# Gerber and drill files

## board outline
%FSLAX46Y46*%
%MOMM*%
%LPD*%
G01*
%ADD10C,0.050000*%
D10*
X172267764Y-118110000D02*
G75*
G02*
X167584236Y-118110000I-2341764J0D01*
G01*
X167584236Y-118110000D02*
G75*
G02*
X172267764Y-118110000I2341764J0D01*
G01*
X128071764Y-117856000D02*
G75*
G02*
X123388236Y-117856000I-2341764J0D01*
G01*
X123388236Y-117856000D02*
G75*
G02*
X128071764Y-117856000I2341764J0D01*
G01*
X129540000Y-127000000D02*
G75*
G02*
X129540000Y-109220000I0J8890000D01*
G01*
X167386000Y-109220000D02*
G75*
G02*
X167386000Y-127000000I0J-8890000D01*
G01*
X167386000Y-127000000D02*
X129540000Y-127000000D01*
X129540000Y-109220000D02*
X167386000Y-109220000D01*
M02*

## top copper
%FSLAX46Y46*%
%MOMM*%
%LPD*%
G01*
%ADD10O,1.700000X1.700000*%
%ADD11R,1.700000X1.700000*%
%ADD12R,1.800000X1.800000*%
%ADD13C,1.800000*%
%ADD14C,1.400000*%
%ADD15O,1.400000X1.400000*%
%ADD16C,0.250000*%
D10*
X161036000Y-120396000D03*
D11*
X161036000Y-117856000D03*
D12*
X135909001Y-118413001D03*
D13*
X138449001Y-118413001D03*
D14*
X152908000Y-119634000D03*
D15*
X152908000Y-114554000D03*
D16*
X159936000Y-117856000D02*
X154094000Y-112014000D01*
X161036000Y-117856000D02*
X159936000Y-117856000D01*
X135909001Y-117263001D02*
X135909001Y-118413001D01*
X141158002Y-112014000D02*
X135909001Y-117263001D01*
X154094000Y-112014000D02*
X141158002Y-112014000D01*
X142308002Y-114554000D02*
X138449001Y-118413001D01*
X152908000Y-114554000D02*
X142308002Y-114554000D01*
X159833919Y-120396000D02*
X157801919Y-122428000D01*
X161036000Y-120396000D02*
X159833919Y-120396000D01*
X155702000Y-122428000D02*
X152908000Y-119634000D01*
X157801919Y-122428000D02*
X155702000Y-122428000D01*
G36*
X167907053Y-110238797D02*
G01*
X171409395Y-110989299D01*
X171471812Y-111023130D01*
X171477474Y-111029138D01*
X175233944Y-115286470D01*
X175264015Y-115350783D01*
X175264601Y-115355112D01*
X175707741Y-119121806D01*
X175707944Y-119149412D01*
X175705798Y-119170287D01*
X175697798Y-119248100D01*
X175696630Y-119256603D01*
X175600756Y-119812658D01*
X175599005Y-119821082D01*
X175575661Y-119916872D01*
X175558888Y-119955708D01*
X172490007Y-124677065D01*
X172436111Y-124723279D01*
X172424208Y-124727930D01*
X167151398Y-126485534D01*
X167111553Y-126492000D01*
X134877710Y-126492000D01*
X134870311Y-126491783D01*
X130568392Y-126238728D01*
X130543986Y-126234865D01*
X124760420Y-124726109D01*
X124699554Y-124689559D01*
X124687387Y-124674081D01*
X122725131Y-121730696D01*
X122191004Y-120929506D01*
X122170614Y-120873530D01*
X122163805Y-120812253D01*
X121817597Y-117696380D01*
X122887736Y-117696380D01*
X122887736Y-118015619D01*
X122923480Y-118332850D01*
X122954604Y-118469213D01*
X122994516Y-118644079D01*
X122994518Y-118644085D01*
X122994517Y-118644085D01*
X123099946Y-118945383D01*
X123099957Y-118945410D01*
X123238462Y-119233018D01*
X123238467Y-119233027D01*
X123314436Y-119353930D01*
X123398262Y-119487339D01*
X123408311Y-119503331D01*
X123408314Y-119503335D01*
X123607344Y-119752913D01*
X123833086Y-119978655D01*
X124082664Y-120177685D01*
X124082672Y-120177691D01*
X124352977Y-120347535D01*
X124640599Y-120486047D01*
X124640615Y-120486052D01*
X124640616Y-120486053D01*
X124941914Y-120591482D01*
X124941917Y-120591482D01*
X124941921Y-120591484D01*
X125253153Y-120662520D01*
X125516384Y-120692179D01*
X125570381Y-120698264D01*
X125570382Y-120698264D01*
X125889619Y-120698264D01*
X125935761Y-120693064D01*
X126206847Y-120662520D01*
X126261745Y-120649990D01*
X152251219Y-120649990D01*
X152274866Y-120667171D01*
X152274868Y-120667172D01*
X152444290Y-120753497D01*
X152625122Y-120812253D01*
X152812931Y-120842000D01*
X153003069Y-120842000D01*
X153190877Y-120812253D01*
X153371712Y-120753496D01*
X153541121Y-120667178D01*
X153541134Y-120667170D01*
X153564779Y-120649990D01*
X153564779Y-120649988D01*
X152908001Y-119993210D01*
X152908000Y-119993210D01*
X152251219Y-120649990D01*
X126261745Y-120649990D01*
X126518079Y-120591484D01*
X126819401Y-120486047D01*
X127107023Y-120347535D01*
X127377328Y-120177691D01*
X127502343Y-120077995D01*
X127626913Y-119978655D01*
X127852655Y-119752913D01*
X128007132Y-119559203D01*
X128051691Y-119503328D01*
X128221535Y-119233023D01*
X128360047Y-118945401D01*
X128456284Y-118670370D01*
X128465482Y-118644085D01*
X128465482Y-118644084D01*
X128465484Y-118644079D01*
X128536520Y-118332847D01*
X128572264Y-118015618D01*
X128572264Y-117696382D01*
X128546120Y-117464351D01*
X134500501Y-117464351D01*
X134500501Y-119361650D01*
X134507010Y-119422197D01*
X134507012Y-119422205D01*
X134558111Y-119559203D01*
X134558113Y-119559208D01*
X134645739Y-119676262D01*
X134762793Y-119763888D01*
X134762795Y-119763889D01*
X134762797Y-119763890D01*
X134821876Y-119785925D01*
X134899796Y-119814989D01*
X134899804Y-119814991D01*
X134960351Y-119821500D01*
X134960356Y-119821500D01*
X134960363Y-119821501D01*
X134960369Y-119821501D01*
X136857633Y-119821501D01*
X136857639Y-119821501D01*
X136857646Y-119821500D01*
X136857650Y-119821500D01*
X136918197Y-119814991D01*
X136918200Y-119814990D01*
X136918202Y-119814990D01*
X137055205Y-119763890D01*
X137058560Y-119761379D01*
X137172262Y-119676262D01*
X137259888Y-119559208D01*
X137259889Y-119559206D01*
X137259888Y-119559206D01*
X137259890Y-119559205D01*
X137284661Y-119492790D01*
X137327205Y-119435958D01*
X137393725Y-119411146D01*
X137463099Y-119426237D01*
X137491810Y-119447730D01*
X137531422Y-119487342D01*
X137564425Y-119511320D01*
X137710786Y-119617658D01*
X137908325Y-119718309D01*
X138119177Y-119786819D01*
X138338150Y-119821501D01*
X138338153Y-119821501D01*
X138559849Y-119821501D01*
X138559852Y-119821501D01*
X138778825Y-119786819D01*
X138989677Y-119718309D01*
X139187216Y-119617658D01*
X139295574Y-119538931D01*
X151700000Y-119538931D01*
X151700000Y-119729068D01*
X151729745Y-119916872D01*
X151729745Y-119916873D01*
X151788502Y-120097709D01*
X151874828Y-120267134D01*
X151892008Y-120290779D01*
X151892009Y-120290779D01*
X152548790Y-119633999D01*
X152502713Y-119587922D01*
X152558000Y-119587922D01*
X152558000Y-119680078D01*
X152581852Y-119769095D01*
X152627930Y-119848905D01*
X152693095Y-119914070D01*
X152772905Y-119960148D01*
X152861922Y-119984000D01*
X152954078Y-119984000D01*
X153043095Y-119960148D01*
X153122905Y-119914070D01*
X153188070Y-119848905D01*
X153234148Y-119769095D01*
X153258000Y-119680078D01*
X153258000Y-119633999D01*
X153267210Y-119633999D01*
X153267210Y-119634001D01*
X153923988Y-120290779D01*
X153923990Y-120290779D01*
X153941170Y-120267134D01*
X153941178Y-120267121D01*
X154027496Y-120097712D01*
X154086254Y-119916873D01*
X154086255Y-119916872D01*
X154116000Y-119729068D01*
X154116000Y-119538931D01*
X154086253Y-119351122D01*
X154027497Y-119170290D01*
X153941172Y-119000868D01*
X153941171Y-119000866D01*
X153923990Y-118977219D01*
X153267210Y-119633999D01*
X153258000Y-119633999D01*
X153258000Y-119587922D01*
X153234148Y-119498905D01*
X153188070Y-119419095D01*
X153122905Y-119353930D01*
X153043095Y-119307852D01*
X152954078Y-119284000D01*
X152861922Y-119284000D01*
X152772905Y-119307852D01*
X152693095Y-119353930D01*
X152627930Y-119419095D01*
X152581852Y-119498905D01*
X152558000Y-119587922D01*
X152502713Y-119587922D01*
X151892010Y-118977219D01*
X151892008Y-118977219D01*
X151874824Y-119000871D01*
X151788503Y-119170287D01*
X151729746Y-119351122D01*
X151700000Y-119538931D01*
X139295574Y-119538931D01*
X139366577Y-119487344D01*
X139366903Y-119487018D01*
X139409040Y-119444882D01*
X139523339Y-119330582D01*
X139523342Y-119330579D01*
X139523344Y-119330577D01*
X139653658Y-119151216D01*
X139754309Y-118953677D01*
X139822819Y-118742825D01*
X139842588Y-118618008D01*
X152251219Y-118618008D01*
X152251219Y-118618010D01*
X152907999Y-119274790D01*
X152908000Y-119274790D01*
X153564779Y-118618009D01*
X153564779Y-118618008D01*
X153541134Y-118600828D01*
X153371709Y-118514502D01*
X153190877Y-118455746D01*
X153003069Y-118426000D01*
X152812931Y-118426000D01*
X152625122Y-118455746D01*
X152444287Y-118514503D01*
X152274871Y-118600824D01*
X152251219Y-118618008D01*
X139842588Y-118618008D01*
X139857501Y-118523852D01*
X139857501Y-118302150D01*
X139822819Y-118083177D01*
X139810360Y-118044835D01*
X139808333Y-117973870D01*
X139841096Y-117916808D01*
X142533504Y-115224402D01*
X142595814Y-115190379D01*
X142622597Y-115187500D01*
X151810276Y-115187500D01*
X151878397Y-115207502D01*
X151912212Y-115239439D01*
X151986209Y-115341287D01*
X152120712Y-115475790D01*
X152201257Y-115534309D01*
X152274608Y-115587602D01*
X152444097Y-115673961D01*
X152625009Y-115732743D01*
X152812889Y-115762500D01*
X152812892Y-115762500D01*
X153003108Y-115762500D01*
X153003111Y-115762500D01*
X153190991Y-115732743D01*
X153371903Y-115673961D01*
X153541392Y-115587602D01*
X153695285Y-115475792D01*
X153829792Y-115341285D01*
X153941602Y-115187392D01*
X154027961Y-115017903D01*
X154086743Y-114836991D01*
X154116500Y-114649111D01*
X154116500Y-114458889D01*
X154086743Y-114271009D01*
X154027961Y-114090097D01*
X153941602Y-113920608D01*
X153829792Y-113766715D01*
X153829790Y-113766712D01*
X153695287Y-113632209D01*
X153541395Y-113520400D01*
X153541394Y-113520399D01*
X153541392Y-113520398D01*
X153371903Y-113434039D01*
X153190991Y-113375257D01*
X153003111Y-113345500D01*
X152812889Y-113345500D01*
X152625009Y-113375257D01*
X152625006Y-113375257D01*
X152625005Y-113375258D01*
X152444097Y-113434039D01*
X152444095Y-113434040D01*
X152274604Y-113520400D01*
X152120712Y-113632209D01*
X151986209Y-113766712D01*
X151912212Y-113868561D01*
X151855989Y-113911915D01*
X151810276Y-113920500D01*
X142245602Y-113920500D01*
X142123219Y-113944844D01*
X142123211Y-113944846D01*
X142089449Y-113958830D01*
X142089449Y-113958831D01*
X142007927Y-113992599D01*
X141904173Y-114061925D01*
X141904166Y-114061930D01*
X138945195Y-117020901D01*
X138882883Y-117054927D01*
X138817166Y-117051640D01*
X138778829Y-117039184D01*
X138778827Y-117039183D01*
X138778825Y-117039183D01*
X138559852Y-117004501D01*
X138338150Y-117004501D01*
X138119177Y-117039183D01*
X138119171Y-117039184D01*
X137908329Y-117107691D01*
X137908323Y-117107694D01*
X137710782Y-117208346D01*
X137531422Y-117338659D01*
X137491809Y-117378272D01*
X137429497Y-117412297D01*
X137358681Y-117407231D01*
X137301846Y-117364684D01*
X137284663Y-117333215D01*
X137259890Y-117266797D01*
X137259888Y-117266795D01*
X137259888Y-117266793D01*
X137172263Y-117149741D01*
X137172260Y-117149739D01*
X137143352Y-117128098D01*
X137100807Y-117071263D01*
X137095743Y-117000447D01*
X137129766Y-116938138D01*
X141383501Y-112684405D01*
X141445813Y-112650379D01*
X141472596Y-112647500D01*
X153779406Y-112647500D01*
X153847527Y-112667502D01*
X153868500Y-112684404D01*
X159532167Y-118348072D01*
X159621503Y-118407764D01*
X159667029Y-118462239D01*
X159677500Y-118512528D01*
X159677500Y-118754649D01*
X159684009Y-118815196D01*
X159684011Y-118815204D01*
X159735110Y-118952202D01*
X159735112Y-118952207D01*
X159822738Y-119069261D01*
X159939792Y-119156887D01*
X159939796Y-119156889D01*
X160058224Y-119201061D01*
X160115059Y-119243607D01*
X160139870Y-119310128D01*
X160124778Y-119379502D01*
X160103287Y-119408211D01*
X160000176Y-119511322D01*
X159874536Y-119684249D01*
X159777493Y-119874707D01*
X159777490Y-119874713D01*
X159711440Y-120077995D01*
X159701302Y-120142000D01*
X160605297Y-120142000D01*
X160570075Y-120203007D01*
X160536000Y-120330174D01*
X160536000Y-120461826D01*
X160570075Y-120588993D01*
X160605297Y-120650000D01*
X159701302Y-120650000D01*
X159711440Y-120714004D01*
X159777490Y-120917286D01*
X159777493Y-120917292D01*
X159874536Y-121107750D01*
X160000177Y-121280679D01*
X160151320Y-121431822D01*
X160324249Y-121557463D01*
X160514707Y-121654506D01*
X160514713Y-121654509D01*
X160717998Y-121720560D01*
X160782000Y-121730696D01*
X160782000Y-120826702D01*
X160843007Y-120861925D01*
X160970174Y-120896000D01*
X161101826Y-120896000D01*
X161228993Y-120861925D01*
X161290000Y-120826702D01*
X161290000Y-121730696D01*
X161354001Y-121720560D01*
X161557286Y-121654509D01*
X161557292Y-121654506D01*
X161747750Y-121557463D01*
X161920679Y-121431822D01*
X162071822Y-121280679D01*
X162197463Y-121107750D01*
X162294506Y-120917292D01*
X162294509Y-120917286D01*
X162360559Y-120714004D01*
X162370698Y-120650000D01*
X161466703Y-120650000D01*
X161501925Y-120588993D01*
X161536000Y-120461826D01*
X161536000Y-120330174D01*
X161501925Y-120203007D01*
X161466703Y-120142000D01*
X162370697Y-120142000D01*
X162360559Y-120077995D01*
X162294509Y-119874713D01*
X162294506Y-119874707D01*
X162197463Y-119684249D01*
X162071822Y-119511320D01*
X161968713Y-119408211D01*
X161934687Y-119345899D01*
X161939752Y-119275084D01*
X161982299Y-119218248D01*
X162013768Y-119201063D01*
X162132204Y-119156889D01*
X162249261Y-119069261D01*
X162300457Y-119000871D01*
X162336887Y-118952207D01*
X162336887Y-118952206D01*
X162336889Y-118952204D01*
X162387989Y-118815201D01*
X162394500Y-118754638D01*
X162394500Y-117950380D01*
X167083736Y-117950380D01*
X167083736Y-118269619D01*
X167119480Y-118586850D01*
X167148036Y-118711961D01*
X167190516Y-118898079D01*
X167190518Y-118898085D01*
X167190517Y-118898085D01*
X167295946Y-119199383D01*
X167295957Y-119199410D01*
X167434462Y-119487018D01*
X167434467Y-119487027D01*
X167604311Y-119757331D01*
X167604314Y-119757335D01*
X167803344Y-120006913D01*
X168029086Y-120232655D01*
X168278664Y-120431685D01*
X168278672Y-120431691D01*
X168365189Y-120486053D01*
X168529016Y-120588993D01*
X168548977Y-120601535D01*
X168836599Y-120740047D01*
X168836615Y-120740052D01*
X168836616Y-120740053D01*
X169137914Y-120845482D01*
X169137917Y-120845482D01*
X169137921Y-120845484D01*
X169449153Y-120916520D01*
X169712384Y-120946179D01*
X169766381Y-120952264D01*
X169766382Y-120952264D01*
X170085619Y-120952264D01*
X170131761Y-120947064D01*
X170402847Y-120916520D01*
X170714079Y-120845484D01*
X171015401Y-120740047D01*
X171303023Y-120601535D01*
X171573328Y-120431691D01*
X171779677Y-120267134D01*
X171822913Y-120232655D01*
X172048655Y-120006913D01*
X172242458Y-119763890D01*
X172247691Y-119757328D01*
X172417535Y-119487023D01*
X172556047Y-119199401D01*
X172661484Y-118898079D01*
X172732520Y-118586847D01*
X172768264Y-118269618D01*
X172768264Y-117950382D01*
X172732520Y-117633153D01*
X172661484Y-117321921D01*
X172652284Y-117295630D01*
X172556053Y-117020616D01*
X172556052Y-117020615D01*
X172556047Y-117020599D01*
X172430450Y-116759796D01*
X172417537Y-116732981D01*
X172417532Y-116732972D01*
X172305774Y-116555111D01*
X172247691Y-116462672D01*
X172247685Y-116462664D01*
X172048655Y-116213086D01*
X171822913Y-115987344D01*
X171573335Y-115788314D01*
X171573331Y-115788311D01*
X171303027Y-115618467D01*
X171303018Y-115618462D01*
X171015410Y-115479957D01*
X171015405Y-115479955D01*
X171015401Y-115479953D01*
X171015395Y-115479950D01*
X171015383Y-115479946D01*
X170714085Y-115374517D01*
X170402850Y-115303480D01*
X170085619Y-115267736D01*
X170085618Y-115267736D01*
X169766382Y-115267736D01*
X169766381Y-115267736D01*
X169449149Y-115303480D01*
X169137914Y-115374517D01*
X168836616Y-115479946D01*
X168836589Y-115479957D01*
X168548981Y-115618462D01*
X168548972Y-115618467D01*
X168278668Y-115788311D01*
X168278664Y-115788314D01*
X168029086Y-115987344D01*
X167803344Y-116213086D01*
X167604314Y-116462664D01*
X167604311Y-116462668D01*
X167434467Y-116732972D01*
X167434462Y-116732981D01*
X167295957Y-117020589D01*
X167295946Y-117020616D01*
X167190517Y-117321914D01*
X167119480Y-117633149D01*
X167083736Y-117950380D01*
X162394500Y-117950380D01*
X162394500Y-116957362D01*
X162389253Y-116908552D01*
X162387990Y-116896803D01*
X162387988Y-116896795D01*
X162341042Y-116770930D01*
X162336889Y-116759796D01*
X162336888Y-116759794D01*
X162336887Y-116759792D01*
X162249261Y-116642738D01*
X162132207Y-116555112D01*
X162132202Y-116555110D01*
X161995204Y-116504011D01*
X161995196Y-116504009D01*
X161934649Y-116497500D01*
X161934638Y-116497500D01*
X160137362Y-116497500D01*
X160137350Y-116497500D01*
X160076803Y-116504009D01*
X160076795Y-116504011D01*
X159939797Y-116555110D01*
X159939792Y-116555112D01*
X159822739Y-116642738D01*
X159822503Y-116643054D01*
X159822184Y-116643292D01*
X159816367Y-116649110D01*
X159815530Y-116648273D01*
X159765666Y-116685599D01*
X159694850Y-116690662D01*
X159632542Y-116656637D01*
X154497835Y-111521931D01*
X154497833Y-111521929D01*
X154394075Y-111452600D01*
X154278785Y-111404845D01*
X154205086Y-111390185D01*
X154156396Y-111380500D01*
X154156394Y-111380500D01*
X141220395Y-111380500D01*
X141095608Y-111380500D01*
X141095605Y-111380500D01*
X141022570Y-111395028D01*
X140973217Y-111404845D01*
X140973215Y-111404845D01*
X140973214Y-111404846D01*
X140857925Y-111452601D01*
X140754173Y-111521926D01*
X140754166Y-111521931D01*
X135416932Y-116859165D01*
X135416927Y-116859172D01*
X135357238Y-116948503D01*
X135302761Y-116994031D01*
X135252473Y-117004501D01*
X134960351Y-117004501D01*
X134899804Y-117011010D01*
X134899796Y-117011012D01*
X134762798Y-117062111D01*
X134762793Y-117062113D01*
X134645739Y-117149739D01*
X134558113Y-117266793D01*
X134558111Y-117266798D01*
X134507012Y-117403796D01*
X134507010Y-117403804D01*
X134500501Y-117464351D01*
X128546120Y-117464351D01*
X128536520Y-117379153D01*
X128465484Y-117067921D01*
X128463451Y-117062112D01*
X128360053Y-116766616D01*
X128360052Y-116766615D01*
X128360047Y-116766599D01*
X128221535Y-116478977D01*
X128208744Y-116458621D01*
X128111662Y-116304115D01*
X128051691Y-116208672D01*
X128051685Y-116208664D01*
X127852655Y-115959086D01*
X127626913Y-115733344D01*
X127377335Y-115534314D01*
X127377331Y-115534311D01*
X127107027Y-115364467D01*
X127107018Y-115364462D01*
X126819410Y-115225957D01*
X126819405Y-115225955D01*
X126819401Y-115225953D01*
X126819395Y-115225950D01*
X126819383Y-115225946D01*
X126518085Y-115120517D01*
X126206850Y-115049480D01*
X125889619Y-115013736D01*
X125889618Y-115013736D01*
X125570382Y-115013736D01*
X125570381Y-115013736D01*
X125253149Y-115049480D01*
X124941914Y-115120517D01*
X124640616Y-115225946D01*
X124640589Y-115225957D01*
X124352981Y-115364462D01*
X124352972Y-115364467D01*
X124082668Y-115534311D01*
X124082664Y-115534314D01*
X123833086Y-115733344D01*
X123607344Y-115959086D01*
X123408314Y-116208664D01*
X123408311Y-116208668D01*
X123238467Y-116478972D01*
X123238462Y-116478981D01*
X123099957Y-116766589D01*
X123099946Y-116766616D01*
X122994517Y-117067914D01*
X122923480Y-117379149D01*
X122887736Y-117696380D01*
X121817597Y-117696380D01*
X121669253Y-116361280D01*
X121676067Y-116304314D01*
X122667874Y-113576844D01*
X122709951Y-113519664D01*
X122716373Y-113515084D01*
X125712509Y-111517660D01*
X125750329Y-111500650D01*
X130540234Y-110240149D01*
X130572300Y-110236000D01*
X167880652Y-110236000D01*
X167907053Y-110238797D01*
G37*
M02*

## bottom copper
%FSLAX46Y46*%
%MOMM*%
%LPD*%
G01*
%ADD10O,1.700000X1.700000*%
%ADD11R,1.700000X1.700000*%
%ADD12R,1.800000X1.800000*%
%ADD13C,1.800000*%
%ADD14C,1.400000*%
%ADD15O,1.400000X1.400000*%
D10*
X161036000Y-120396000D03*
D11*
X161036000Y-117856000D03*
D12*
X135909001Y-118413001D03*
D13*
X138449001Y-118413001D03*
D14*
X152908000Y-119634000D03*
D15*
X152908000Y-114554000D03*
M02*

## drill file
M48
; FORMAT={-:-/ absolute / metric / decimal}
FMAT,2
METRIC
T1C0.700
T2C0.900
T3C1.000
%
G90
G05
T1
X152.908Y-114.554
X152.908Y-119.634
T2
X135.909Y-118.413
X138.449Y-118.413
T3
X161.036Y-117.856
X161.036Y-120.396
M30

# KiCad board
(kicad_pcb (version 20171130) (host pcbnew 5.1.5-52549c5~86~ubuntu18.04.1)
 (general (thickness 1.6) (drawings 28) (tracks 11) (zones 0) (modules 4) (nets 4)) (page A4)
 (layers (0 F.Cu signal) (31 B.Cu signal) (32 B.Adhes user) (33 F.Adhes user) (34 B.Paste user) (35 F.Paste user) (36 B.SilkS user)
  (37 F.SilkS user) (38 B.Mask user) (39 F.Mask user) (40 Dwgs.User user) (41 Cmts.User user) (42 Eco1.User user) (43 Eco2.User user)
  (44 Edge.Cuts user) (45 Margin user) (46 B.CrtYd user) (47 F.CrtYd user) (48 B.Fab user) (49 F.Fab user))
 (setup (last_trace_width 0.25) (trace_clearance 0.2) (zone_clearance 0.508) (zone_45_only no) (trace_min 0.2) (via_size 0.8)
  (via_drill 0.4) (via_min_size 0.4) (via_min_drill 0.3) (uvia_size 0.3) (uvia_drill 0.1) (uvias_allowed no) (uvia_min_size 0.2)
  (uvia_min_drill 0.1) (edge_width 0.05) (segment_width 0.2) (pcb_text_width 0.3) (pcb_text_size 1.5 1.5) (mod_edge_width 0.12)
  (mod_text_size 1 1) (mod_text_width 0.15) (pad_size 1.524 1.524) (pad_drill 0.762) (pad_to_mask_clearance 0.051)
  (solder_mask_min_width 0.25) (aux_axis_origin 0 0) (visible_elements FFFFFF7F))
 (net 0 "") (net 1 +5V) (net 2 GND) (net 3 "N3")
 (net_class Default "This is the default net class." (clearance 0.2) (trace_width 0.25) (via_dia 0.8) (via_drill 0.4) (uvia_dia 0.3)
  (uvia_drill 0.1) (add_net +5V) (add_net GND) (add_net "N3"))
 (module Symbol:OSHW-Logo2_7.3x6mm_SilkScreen (layer B.Cu) (at 146.558 121.158)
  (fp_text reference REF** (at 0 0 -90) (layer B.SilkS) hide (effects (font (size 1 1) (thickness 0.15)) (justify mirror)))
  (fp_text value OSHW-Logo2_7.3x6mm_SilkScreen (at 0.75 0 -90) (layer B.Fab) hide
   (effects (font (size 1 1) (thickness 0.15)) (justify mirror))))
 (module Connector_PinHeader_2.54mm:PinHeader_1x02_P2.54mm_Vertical (layer F.Cu) (at 161.036 117.856)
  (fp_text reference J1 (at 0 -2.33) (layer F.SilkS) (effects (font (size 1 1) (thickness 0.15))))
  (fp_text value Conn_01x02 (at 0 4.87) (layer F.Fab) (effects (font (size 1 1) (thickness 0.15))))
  (pad 2 thru_hole oval (at 0 2.54) (size 1.7 1.7) (drill 1) (layers *.Cu *.Mask) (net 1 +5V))
  (pad 1 thru_hole rect (at 0 0) (size 1.7 1.7) (drill 1) (layers *.Cu *.Mask) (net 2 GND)))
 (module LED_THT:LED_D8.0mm (layer F.Cu) (at 135.909001 118.413001)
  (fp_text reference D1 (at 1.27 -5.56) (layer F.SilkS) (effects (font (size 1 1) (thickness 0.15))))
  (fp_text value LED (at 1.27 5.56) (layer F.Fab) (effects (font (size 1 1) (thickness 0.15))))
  (pad 1 thru_hole rect (at 0 0) (size 1.8 1.8) (drill 0.9) (layers *.Cu *.Mask) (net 2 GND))
  (pad 2 thru_hole circle (at 2.54 0) (size 1.8 1.8) (drill 0.9) (layers *.Cu *.Mask) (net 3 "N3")))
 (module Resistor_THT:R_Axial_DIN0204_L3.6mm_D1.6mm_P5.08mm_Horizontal (layer F.Cu) (at 152.908 119.634 90)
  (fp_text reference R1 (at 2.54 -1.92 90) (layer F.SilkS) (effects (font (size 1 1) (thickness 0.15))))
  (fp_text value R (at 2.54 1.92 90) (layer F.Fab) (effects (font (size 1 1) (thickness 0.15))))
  (pad 1 thru_hole circle (at 0 0 90) (size 1.4 1.4) (drill 0.7) (layers *.Cu *.Mask) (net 1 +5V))
  (pad 2 thru_hole oval (at 5.08 0 90) (size 1.4 1.4) (drill 0.7) (layers *.Cu *.Mask) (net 3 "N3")))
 (gr_circle (center 169.926 118.11) (end 171.45 119.888) (layer Edge.Cuts) (width 0.05))
 (gr_circle (center 125.73 117.856) (end 127.254 119.634) (layer Edge.Cuts) (width 0.05))
 (gr_arc (start 129.54 118.11) (end 129.54 109.22) (angle -180) (layer Edge.Cuts) (width 0.05))
 (gr_arc (start 167.386 118.11) (end 167.386 127) (angle -180) (layer Edge.Cuts) (width 0.05))
 (gr_line (start 167.386 127) (end 129.54 127) (layer Edge.Cuts) (width 0.05))
 (gr_line (start 129.54 109.22) (end 167.386 109.22) (layer Edge.Cuts) (width 0.05))
 (segment (start 159.936 117.856) (end 154.094 112.014) (width 0.25) (layer F.Cu) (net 2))
 (segment (start 161.036 117.856) (end 159.936 117.856) (width 0.25) (layer F.Cu) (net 2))
 (segment (start 135.909001 117.263001) (end 135.909001 118.413001) (width 0.25) (layer F.Cu) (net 2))
 (segment (start 141.158002 112.014) (end 135.909001 117.263001) (width 0.25) (layer F.Cu) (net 2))
 (segment (start 154.094 112.014) (end 141.158002 112.014) (width 0.25) (layer F.Cu) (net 2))
 (segment (start 142.308002 114.554) (end 138.449001 118.413001) (width 0.25) (layer F.Cu) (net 3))
 (segment (start 152.908 114.554) (end 142.308002 114.554) (width 0.25) (layer F.Cu) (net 3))
 (segment (start 159.833919 120.396) (end 157.801919 122.428) (width 0.25) (layer F.Cu) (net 1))
 (segment (start 161.036 120.396) (end 159.833919 120.396) (width 0.25) (layer F.Cu) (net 1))
 (segment (start 155.702 122.428) (end 152.908 119.634) (width 0.25) (layer F.Cu) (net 1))
 (segment (start 157.801919 122.428) (end 155.702 122.428) (width 0.25) (layer F.Cu) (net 1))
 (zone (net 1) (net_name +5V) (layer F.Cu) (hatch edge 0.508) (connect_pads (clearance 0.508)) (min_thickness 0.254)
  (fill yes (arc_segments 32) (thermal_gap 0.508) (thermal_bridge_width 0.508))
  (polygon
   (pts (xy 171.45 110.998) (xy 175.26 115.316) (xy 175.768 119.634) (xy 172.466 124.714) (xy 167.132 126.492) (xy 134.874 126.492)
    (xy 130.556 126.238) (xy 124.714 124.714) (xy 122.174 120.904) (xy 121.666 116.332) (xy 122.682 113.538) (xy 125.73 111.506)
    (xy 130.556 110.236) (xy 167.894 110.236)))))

